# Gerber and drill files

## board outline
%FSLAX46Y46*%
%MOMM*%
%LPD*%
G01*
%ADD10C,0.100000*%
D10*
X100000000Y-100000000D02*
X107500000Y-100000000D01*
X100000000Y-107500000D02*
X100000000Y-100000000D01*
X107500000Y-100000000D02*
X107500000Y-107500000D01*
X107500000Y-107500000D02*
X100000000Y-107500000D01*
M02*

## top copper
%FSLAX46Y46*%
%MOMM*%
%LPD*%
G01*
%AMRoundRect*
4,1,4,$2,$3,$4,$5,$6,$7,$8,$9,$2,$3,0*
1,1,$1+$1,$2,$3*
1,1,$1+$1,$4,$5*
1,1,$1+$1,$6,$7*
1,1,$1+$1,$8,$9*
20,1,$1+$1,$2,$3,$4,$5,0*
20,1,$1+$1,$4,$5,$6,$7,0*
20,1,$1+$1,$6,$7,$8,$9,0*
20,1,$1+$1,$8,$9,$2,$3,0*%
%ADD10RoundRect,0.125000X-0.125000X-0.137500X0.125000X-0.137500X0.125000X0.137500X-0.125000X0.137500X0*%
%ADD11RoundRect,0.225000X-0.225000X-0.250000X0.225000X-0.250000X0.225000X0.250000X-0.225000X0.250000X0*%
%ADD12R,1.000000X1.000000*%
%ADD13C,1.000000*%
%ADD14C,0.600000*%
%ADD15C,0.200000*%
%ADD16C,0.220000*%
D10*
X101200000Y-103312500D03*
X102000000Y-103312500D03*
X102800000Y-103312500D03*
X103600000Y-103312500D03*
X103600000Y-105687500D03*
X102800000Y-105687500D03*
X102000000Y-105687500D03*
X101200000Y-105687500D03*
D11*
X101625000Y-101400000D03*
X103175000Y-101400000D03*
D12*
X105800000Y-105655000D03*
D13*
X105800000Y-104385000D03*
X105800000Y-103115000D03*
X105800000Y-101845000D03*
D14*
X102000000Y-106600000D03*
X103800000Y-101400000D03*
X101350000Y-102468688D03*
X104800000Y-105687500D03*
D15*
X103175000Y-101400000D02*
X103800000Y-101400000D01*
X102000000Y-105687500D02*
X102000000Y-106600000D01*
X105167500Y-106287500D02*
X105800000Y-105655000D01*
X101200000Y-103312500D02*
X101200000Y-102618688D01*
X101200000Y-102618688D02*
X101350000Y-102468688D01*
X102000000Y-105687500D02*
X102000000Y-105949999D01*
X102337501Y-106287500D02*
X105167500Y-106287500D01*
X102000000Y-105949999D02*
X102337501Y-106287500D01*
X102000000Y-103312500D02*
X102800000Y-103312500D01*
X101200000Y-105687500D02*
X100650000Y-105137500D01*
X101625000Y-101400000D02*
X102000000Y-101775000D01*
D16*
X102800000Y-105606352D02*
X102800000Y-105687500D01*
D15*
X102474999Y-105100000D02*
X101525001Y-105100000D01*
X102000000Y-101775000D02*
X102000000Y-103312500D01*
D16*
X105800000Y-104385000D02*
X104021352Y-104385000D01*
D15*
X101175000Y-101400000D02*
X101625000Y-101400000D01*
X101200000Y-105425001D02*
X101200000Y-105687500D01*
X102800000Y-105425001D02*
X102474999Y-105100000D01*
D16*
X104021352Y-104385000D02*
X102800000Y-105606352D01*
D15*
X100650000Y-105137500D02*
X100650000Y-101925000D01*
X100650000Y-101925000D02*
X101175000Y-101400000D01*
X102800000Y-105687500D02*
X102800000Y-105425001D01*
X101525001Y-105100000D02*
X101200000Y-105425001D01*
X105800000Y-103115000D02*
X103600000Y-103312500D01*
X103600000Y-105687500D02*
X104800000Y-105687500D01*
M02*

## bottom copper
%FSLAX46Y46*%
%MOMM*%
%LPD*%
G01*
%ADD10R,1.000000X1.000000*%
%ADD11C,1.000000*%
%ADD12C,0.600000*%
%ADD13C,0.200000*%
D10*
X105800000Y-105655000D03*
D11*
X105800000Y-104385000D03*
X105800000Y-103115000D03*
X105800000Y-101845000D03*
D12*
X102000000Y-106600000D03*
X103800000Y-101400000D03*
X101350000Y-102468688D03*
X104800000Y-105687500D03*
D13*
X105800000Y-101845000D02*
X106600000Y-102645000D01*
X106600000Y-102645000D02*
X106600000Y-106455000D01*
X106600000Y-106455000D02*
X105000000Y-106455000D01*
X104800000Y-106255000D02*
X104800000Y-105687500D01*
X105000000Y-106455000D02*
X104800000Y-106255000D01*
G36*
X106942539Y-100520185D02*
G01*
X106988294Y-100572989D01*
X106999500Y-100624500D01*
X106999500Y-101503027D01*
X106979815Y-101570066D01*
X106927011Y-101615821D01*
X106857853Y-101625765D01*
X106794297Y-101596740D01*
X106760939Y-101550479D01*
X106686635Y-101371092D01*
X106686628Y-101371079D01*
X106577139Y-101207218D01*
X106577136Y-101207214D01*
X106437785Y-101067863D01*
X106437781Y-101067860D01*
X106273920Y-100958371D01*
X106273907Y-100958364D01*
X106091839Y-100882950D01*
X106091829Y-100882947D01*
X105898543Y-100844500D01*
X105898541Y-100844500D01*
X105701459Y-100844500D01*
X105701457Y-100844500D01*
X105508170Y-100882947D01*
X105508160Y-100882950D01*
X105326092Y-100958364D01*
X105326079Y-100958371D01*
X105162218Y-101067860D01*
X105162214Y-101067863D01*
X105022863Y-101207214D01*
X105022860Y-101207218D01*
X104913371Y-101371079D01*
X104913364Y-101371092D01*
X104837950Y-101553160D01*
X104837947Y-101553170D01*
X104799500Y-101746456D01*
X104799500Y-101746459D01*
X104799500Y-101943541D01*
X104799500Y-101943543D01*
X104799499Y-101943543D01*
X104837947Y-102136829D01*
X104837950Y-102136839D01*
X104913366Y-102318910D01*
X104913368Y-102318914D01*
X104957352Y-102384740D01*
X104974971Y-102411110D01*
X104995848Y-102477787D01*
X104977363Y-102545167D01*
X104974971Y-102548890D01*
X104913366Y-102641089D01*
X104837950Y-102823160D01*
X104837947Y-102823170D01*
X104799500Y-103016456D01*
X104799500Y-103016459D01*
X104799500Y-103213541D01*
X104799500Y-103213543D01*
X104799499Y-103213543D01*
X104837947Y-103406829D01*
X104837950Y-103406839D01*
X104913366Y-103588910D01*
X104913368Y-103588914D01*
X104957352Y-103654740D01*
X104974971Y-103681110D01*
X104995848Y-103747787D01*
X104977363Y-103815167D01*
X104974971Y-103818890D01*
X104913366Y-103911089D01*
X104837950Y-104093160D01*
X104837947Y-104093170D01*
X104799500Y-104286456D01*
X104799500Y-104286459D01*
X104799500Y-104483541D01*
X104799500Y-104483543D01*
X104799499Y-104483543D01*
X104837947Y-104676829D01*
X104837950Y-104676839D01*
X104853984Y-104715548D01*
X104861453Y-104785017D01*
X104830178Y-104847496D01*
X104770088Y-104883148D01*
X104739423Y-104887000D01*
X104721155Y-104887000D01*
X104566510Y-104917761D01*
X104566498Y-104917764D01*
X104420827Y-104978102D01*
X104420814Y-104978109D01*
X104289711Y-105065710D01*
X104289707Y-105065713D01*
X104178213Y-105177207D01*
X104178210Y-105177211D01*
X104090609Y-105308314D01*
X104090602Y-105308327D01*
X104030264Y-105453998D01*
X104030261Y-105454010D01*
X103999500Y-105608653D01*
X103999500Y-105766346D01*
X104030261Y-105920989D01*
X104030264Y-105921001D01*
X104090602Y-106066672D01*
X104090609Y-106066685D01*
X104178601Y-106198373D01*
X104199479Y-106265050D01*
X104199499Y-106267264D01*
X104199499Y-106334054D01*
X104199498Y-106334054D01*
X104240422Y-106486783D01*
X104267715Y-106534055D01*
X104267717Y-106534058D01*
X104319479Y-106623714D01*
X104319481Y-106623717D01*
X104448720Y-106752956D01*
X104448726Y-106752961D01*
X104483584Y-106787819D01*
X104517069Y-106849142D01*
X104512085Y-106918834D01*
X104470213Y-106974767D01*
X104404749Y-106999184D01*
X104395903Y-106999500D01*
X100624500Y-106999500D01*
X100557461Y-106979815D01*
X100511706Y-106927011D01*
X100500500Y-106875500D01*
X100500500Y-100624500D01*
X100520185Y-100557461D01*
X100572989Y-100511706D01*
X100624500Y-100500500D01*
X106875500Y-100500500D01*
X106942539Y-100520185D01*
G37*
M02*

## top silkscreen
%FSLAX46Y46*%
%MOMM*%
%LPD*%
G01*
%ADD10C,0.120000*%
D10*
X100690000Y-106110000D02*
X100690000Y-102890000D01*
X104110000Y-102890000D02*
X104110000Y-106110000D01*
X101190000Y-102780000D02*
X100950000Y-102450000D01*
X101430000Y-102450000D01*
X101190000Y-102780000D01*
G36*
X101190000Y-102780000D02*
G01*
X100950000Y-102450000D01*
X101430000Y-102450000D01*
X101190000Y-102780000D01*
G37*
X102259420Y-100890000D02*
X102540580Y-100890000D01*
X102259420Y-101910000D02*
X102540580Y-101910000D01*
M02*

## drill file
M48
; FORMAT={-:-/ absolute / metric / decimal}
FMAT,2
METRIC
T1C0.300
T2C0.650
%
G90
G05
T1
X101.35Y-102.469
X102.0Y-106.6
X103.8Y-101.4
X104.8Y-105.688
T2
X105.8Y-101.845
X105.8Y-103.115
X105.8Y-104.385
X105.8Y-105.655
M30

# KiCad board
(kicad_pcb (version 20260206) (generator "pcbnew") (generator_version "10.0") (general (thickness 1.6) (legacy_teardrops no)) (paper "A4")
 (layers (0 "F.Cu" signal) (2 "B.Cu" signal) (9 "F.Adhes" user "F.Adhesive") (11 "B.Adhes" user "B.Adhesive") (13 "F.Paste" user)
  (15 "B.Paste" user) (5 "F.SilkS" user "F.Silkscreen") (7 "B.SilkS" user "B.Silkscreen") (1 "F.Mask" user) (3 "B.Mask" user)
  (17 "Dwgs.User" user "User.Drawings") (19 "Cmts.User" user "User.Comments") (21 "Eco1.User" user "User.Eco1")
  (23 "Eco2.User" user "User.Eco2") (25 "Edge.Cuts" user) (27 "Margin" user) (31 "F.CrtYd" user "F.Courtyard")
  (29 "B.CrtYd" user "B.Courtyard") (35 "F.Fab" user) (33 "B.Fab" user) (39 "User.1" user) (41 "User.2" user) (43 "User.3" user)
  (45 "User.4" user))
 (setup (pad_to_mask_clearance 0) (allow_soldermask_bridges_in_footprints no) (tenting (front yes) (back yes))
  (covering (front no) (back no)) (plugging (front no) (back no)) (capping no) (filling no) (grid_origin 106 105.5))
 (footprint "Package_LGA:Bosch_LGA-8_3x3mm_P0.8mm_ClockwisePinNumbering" (layer "F.Cu") (at 102.4 104.5)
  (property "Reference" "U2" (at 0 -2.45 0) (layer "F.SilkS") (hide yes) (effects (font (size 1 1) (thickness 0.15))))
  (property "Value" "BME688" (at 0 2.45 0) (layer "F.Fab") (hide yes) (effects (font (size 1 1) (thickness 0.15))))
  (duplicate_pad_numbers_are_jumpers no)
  (fp_line (start -1.71 1.61) (end -1.71 -1.61) (stroke (width 0.12) (type solid)) (layer "F.SilkS"))
  (fp_line (start 1.71 -1.61) (end 1.71 1.61) (stroke (width 0.12) (type solid)) (layer "F.SilkS"))
  (fp_poly (pts (xy -1.21 -1.72) (xy -1.45 -2.05) (xy -0.97 -2.05)) (stroke (width 0.12) (type solid)) (fill yes) (layer "F.SilkS"))
  (pad "1" smd roundrect (at -1.2 -1.1875) (size 0.5 0.525) (layers "F.Cu" "F.Mask" "F.Paste") (roundrect_rratio 0.25) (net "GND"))
  (pad "2" smd roundrect (at -0.4 -1.1875) (size 0.5 0.525) (layers "F.Cu" "F.Mask" "F.Paste") (roundrect_rratio 0.25) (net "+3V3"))
  (pad "3" smd roundrect (at 0.4 -1.1875) (size 0.5 0.525) (layers "F.Cu" "F.Mask" "F.Paste") (roundrect_rratio 0.25) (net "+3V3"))
  (pad "4" smd roundrect (at 1.2 -1.1875) (size 0.5 0.525) (layers "F.Cu" "F.Mask" "F.Paste") (roundrect_rratio 0.25) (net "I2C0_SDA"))
  (pad "5" smd roundrect (at 1.2 1.1875) (size 0.5 0.525) (layers "F.Cu" "F.Mask" "F.Paste") (roundrect_rratio 0.25) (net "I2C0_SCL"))
  (pad "6" smd roundrect (at 0.4 1.1875) (size 0.5 0.525) (layers "F.Cu" "F.Mask" "F.Paste") (roundrect_rratio 0.25) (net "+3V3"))
  (pad "7" smd roundrect (at -0.4 1.1875) (size 0.5 0.525) (layers "F.Cu" "F.Mask" "F.Paste") (roundrect_rratio 0.25) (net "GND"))
  (pad "8" smd roundrect (at -1.2 1.1875) (size 0.5 0.525) (layers "F.Cu" "F.Mask" "F.Paste") (roundrect_rratio 0.25) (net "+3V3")))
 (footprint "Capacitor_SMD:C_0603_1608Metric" (layer "F.Cu") (at 102.4 101.4)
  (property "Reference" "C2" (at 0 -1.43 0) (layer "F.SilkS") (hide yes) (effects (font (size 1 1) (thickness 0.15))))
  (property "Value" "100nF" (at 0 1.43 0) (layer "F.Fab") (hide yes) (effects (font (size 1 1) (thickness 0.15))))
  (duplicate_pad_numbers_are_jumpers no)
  (fp_line (start -0.14058 -0.51) (end 0.14058 -0.51) (stroke (width 0.12) (type solid)) (layer "F.SilkS"))
  (fp_line (start -0.14058 0.51) (end 0.14058 0.51) (stroke (width 0.12) (type solid)) (layer "F.SilkS"))
  (pad "1" smd roundrect (at -0.775 0) (size 0.9 0.95) (layers "F.Cu" "F.Mask" "F.Paste") (roundrect_rratio 0.25) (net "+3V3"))
  (pad "2" smd roundrect (at 0.775 0) (size 0.9 0.95) (layers "F.Cu" "F.Mask" "F.Paste") (roundrect_rratio 0.25) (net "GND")))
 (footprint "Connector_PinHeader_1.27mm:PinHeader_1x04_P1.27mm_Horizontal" (layer "B.Cu") (at 105.8 105.655)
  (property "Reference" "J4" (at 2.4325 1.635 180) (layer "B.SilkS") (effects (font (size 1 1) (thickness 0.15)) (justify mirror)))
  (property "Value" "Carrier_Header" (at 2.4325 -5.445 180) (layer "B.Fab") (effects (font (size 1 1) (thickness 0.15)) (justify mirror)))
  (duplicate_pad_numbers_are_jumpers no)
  (pad "1" thru_hole rect (at 0 0) (size 1 1) (drill 0.65) (layers "*.Cu" "*.Mask") (remove_unused_layers no) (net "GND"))
  (pad "2" thru_hole circle (at 0 -1.27) (size 1 1) (drill 0.65) (layers "*.Cu" "*.Mask") (remove_unused_layers no) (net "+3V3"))
  (pad "3" thru_hole circle (at 0 -2.54) (size 1 1) (drill 0.65) (layers "*.Cu" "*.Mask") (remove_unused_layers no) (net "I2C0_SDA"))
  (pad "4" thru_hole circle (at 0 -3.81) (size 1 1) (drill 0.65) (layers "*.Cu" "*.Mask") (remove_unused_layers no) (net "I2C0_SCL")))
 (gr_line (start 100 100) (end 107.5 100) (stroke (width 0.1) (type default)) (layer "Edge.Cuts"))
 (gr_line (start 100 107.5) (end 100 100) (stroke (width 0.1) (type default)) (layer "Edge.Cuts"))
 (gr_line (start 107.5 100) (end 107.5 107.5) (stroke (width 0.1) (type default)) (layer "Edge.Cuts"))
 (gr_line (start 107.5 107.5) (end 100 107.5) (stroke (width 0.1) (type default)) (layer "Edge.Cuts"))
 (segment (start 103.175 101.4) (end 103.8 101.4) (width 0.2) (layer "F.Cu") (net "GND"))
 (segment (start 102 105.6875) (end 102 106.6) (width 0.2) (layer "F.Cu") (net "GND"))
 (segment (start 105.1675 106.2875) (end 105.8 105.655) (width 0.2) (layer "F.Cu") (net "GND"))
 (segment (start 101.2 103.3125) (end 101.2 102.618688) (width 0.2) (layer "F.Cu") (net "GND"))
 (segment (start 101.2 102.618688) (end 101.35 102.468688) (width 0.2) (layer "F.Cu") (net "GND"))
 (segment (start 102 105.6875) (end 102 105.949999) (width 0.2) (layer "F.Cu") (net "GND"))
 (segment (start 102.337501 106.2875) (end 105.1675 106.2875) (width 0.2) (layer "F.Cu") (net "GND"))
 (segment (start 102 105.949999) (end 102.337501 106.2875) (width 0.2) (layer "F.Cu") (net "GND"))
 (via (at 102 106.6) (size 0.6) (drill 0.3) (layers "F.Cu" "B.Cu") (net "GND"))
 (via (at 103.8 101.4) (size 0.6) (drill 0.3) (layers "F.Cu" "B.Cu") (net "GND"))
 (via (at 101.35 102.468688) (size 0.6) (drill 0.3) (layers "F.Cu" "B.Cu") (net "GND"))
 (segment (start 102 103.3125) (end 102.8 103.3125) (width 0.2) (layer "F.Cu") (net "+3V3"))
 (segment (start 101.2 105.6875) (end 100.65 105.1375) (width 0.2) (layer "F.Cu") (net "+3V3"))
 (segment (start 101.625 101.4) (end 102 101.775) (width 0.2) (layer "F.Cu") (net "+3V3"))
 (segment (start 102.8 105.606352) (end 102.8 105.6875) (width 0.22) (layer "F.Cu") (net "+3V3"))
 (segment (start 102.474999 105.1) (end 101.525001 105.1) (width 0.2) (layer "F.Cu") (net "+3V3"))
 (segment (start 102 101.775) (end 102 103.3125) (width 0.2) (layer "F.Cu") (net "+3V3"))
 (segment (start 105.8 104.385) (end 104.021352 104.385) (width 0.22) (layer "F.Cu") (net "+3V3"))
 (segment (start 101.175 101.4) (end 101.625 101.4) (width 0.2) (layer "F.Cu") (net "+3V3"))
 (segment (start 101.2 105.425001) (end 101.2 105.6875) (width 0.2) (layer "F.Cu") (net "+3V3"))
 (segment (start 102.8 105.425001) (end 102.474999 105.1) (width 0.2) (layer "F.Cu") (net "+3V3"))
 (segment (start 104.021352 104.385) (end 102.8 105.606352) (width 0.22) (layer "F.Cu") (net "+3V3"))
 (segment (start 100.65 105.1375) (end 100.65 101.925) (width 0.2) (layer "F.Cu") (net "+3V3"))
 (segment (start 100.65 101.925) (end 101.175 101.4) (width 0.2) (layer "F.Cu") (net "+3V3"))
 (segment (start 102.8 105.6875) (end 102.8 105.425001) (width 0.2) (layer "F.Cu") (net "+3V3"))
 (segment (start 101.525001 105.1) (end 101.2 105.425001) (width 0.2) (layer "F.Cu") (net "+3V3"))
 (segment (start 105.8 103.115) (end 103.6 103.3125) (width 0.2) (layer "F.Cu") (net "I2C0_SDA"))
 (segment (start 103.6 105.6875) (end 104.8 105.6875) (width 0.2) (layer "F.Cu") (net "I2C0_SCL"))
 (via (at 104.8 105.6875) (size 0.6) (drill 0.3) (layers "F.Cu" "B.Cu") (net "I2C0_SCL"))
 (segment (start 105.8 101.845) (end 106.6 102.645) (width 0.2) (layer "B.Cu") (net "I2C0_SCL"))
 (segment (start 106.6 102.645) (end 106.6 106.455) (width 0.2) (layer "B.Cu") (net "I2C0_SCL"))
 (segment (start 106.6 106.455) (end 105 106.455) (width 0.2) (layer "B.Cu") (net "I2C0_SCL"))
 (segment (start 104.8 106.255) (end 104.8 105.6875) (width 0.2) (layer "B.Cu") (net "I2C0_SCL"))
 (segment (start 105 106.455) (end 104.8 106.255) (width 0.2) (layer "B.Cu") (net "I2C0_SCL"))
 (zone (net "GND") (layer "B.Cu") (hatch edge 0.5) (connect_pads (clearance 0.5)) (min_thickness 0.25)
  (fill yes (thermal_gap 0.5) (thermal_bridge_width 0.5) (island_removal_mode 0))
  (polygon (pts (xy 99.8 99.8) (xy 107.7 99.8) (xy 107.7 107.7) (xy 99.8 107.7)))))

